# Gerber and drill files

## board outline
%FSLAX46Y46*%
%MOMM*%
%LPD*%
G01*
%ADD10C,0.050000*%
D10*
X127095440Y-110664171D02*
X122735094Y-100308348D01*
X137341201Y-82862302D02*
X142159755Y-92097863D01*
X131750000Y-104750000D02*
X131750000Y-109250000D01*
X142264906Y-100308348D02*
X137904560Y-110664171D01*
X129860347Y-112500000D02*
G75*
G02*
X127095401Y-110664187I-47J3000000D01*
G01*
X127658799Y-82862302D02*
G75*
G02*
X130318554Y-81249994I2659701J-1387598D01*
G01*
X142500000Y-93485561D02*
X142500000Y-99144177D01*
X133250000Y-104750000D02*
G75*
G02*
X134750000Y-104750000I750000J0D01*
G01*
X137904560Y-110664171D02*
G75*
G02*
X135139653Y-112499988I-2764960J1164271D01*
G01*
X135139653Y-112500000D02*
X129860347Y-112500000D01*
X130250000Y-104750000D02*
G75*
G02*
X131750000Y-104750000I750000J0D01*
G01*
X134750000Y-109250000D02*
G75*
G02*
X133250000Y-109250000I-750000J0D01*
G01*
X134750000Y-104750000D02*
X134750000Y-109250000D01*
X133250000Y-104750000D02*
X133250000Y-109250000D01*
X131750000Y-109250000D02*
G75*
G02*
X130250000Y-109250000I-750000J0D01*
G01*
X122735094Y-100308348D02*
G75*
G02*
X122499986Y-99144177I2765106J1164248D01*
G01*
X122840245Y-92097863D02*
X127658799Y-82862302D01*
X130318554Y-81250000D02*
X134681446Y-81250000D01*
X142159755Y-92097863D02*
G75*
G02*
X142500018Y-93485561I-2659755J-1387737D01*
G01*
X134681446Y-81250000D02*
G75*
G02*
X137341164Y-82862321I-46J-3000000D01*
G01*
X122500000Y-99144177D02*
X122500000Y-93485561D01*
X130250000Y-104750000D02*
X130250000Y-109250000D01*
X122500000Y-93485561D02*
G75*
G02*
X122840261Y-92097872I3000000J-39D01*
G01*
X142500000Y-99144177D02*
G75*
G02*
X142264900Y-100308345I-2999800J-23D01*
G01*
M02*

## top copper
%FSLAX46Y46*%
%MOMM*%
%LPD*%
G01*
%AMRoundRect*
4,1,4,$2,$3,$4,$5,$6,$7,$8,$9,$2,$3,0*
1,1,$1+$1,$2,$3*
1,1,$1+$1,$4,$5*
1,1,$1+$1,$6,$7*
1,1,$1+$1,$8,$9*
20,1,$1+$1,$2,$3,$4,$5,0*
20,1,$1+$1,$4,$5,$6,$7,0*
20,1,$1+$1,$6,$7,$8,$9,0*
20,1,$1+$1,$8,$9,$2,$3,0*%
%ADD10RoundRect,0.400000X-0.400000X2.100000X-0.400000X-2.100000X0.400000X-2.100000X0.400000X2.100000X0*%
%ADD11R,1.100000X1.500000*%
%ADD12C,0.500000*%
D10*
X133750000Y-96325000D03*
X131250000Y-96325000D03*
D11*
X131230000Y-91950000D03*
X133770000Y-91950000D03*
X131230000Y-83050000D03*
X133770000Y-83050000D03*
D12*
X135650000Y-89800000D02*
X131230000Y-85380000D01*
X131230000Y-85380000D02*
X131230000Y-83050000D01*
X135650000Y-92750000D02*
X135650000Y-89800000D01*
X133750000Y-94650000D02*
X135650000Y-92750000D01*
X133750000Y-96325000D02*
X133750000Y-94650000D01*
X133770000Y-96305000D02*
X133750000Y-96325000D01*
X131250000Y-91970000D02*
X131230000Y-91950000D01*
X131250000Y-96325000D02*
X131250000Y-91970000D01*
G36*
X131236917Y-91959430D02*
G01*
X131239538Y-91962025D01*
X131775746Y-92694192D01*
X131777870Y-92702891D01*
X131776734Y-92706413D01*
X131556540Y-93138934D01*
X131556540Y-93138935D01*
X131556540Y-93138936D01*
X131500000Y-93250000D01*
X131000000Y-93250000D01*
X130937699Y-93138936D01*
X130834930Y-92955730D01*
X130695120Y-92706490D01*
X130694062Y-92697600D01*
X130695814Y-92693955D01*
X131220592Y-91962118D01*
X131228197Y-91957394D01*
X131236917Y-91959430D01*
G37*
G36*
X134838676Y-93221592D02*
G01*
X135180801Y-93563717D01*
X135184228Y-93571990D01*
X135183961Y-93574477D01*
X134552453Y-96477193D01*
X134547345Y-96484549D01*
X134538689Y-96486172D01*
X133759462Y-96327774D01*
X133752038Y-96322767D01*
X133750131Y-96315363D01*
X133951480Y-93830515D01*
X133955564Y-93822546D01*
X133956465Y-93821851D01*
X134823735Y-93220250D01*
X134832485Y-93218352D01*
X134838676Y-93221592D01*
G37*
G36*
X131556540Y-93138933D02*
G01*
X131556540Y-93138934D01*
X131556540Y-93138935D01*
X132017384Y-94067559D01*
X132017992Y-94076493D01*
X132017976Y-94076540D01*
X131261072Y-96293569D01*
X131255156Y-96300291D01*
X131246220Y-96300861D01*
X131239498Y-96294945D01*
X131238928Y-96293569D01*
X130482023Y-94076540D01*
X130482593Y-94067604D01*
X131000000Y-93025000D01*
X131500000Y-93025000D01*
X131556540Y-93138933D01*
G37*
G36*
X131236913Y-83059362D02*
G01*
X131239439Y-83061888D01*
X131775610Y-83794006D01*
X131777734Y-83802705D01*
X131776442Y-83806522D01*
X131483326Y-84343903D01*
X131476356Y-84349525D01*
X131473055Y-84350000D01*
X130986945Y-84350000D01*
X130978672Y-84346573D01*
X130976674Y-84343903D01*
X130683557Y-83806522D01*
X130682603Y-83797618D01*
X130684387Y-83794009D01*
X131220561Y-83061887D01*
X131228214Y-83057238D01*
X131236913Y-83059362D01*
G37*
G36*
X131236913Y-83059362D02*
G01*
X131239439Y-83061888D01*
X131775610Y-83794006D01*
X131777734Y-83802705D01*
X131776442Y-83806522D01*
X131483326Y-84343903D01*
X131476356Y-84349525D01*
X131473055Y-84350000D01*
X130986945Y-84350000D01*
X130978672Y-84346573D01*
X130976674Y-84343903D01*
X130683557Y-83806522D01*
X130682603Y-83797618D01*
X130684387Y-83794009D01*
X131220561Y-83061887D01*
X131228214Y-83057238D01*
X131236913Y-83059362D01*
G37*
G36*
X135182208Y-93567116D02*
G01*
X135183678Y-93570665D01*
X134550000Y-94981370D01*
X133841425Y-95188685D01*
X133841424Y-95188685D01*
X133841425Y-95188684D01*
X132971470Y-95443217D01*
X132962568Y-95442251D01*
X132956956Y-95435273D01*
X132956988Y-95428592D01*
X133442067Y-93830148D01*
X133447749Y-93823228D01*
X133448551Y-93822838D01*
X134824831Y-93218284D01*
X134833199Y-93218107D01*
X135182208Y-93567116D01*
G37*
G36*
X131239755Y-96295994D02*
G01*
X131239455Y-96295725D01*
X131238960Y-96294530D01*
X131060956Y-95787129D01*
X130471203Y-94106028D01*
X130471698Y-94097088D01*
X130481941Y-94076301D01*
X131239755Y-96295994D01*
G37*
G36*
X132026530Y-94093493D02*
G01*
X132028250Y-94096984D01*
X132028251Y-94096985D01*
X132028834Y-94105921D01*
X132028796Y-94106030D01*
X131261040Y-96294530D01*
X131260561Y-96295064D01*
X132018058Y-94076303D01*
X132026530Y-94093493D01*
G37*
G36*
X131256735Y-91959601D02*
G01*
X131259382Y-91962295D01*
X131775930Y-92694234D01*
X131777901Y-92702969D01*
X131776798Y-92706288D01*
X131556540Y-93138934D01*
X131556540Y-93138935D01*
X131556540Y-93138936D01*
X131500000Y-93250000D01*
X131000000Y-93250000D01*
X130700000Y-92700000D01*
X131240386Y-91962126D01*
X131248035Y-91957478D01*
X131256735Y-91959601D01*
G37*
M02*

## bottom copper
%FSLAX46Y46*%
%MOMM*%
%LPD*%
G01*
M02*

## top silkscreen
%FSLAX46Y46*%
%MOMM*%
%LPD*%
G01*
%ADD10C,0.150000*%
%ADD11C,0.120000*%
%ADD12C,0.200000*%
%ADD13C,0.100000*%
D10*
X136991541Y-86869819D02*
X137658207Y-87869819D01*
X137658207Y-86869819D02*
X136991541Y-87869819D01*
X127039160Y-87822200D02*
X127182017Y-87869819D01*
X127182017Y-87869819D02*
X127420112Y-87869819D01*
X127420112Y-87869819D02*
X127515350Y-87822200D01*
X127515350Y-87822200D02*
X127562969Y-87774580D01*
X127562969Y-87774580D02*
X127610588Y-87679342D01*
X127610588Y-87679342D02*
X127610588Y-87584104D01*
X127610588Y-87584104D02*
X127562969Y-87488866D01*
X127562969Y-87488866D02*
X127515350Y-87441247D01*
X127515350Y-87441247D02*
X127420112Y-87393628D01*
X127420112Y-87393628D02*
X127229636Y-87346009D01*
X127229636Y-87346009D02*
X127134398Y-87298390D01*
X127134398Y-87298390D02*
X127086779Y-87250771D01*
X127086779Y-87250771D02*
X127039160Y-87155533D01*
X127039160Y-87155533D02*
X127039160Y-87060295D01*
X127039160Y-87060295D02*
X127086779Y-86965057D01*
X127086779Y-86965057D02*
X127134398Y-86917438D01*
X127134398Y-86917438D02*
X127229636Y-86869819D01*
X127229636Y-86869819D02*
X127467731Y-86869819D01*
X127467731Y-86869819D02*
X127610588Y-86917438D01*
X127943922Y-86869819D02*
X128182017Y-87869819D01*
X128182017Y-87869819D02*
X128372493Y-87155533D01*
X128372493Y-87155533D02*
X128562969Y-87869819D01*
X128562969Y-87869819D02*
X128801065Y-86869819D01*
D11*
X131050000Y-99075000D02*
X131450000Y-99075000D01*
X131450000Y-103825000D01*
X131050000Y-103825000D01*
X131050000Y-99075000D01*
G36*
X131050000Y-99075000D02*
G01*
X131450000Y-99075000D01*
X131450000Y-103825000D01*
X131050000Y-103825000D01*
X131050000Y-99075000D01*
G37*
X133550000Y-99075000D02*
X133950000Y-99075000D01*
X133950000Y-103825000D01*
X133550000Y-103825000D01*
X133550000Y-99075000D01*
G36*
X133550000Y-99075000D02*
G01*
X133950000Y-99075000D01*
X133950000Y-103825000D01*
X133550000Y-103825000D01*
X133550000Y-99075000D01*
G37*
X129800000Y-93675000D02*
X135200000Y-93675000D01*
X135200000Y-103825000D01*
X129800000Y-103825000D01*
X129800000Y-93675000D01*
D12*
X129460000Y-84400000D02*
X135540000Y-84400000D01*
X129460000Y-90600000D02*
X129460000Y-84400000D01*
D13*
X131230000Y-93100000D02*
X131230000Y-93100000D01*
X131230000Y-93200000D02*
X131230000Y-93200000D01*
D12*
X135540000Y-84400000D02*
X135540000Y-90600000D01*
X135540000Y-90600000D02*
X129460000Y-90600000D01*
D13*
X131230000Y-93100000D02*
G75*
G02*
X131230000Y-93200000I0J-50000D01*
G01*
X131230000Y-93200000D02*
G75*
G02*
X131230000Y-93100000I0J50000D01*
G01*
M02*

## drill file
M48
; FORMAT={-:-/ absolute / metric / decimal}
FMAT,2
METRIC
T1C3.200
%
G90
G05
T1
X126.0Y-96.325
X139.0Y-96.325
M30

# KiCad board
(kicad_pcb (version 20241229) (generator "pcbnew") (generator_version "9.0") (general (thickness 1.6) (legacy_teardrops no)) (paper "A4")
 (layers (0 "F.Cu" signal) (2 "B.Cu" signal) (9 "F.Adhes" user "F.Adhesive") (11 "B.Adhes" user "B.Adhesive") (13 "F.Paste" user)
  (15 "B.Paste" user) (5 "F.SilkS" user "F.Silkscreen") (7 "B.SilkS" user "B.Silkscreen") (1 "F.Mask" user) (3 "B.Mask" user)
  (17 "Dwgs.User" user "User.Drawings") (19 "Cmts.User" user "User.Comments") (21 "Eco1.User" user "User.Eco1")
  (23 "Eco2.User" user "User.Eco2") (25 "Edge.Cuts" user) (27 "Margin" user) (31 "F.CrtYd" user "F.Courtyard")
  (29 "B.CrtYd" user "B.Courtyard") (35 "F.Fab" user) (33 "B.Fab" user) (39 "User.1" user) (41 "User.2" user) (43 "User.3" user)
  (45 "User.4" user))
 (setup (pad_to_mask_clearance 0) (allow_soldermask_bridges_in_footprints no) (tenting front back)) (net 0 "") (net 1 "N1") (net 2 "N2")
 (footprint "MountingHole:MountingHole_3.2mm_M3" (layer "F.Cu") (at 139 96.325)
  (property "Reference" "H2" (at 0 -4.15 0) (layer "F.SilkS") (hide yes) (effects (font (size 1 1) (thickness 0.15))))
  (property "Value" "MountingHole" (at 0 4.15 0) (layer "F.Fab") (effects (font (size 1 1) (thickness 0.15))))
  (pad "" np_thru_hole circle (at 0 0) (size 3.2 3.2) (drill 3.2) (layers "*.Cu" "*.Mask")))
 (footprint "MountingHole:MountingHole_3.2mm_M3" (layer "F.Cu") (at 126 96.325)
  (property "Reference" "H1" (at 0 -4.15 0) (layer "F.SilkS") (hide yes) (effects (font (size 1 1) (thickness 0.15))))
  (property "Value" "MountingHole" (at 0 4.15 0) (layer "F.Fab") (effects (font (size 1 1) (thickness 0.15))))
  (pad "" np_thru_hole circle (at 0 0) (size 3.2 3.2) (drill 3.2) (layers "*.Cu" "*.Mask")))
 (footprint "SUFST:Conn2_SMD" (layer "F.Cu") (at 132.5 96.325 180)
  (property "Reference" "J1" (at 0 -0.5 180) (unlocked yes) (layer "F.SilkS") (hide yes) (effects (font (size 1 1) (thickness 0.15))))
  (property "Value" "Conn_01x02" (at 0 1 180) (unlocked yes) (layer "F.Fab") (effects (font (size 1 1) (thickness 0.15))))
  (fp_rect (start 1.05 -7.5) (end 1.45 -2.75) (stroke (width 0.12) (type solid)) (fill yes) (layer "F.SilkS"))
  (fp_rect (start -1.45 -7.5) (end -1.05 -2.75) (stroke (width 0.12) (type solid)) (fill yes) (layer "F.SilkS"))
  (fp_rect (start -2.7 -7.5) (end 2.7 2.65) (stroke (width 0.12) (type default)) (fill no) (layer "F.SilkS"))
  (pad "1" smd roundrect (at -1.25 0 270) (size 5 1.6) (layers "F.Cu" "F.Mask" "F.Paste") (roundrect_rratio 0.25) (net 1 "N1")
   (thermal_bridge_angle 45)
   (teardrops (best_length_ratio 0.5) (max_length 1) (best_width_ratio 1) (max_width 2) (curved_edges no) (filter_ratio 0.9) (enabled yes)
    (allow_two_segments yes) (prefer_zone_connections yes)))
  (pad "2" smd roundrect (at 1.25 0 270) (size 5 1.6) (layers "F.Cu" "F.Mask" "F.Paste") (roundrect_rratio 0.25) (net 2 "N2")
   (thermal_bridge_angle 45)
   (teardrops (best_length_ratio 0.5) (max_length 1) (best_width_ratio 1) (max_width 2) (curved_edges no) (filter_ratio 0.9) (enabled yes)
    (allow_two_segments yes) (prefer_zone_connections yes))))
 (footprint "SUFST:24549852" (layer "F.Cu") (at 132.5 87.5)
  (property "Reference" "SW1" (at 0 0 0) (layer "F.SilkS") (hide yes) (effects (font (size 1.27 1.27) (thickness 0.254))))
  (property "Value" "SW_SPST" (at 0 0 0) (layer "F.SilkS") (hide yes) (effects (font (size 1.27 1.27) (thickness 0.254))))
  (fp_line (start -3.04 -3.1) (end 3.04 -3.1) (stroke (width 0.2) (type solid)) (layer "F.SilkS"))
  (fp_line (start -3.04 3.1) (end -3.04 -3.1) (stroke (width 0.2) (type solid)) (layer "F.SilkS"))
  (fp_line (start -1.27 5.6) (end -1.27 5.6) (stroke (width 0.1) (type solid)) (layer "F.SilkS"))
  (fp_line (start -1.27 5.7) (end -1.27 5.7) (stroke (width 0.1) (type solid)) (layer "F.SilkS"))
  (fp_line (start 3.04 -3.1) (end 3.04 3.1) (stroke (width 0.2) (type solid)) (layer "F.SilkS"))
  (fp_line (start 3.04 3.1) (end -3.04 3.1) (stroke (width 0.2) (type solid)) (layer "F.SilkS"))
  (fp_arc (start -1.27 5.6) (mid -1.22 5.65) (end -1.27 5.7) (stroke (width 0.1) (type solid)) (layer "F.SilkS"))
  (fp_arc (start -1.27 5.7) (mid -1.32 5.65) (end -1.27 5.6) (stroke (width 0.1) (type solid)) (layer "F.SilkS"))
  (pad "A1" smd rect (at -1.27 4.45) (size 1.1 1.5) (layers "F.Cu" "F.Mask" "F.Paste") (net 2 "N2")
   (teardrops (best_length_ratio 0.5) (max_length 1) (best_width_ratio 1) (max_width 2) (curved_edges no) (filter_ratio 0.9) (enabled yes)
    (allow_two_segments yes) (prefer_zone_connections yes)))
  (pad "A2" smd rect (at 1.27 4.45) (size 1.1 1.5) (layers "F.Cu" "F.Mask" "F.Paste")
   (teardrops (best_length_ratio 0.5) (max_length 1) (best_width_ratio 1) (max_width 2) (curved_edges no) (filter_ratio 0.9) (enabled yes)
    (allow_two_segments yes) (prefer_zone_connections yes)))
  (pad "B1" smd rect (at -1.27 -4.45) (size 1.1 1.5) (layers "F.Cu" "F.Mask" "F.Paste") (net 1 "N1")
   (teardrops (best_length_ratio 0.5) (max_length 1) (best_width_ratio 1) (max_width 2) (curved_edges no) (filter_ratio 0.9) (enabled yes)
    (allow_two_segments yes) (prefer_zone_connections yes)))
  (pad "B2" smd rect (at 1.27 -4.45) (size 1.1 1.5) (layers "F.Cu" "F.Mask" "F.Paste")
   (teardrops (best_length_ratio 0.5) (max_length 1) (best_width_ratio 1) (max_width 2) (curved_edges no) (filter_ratio 0.9) (enabled yes)
    (allow_two_segments yes) (prefer_zone_connections yes))))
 (gr_line (start 127.09544 110.664171) (end 122.735094 100.308348) (stroke (width 0.05) (type default)) (layer "Edge.Cuts"))
 (gr_line (start 137.341201 82.862302) (end 142.159755 92.097863) (stroke (width 0.05) (type default)) (layer "Edge.Cuts"))
 (gr_line (start 131.75 104.75) (end 131.75 109.25) (stroke (width 0.05) (type default)) (layer "Edge.Cuts"))
 (gr_line (start 142.264906 100.308348) (end 137.90456 110.664171) (stroke (width 0.05) (type default)) (layer "Edge.Cuts"))
 (gr_arc (start 129.860347 112.5) (mid 128.200906 111.999251) (end 127.09544 110.664171) (stroke (width 0.05) (type default))
  (layer "Edge.Cuts"))
 (gr_arc (start 127.658799 82.862302) (mid 128.763412 81.68453) (end 130.318554 81.25) (stroke (width 0.05) (type default))
  (layer "Edge.Cuts"))
 (gr_line (start 142.5 93.485561) (end 142.5 99.144177) (stroke (width 0.05) (type default)) (layer "Edge.Cuts"))
 (gr_arc (start 133.25 104.75) (mid 134 104) (end 134.75 104.75) (stroke (width 0.05) (type default)) (layer "Edge.Cuts"))
 (gr_arc (start 137.90456 110.664171) (mid 136.79909 111.999234) (end 135.139653 112.5) (stroke (width 0.05) (type default))
  (layer "Edge.Cuts"))
 (gr_line (start 135.139653 112.5) (end 129.860347 112.5) (stroke (width 0.05) (type default)) (layer "Edge.Cuts"))
 (gr_arc (start 130.25 104.75) (mid 131 104) (end 131.75 104.75) (stroke (width 0.05) (type default)) (layer "Edge.Cuts"))
 (gr_arc (start 134.75 109.25) (mid 134 110) (end 133.25 109.25) (stroke (width 0.05) (type default)) (layer "Edge.Cuts"))
 (gr_line (start 134.75 104.75) (end 134.75 109.25) (stroke (width 0.05) (type default)) (layer "Edge.Cuts"))
 (gr_line (start 133.25 104.75) (end 133.25 109.25) (stroke (width 0.05) (type default)) (layer "Edge.Cuts"))
 (gr_arc (start 131.75 109.25) (mid 131 110) (end 130.25 109.25) (stroke (width 0.05) (type default)) (layer "Edge.Cuts"))
 (gr_arc (start 122.735094 100.308348) (mid 122.559365 99.738012) (end 122.5 99.144177) (stroke (width 0.05) (type default))
  (layer "Edge.Cuts"))
 (gr_line (start 122.840245 92.097863) (end 127.658799 82.862302) (stroke (width 0.05) (type default)) (layer "Edge.Cuts"))
 (gr_line (start 130.318554 81.25) (end 134.681446 81.25) (stroke (width 0.05) (type default)) (layer "Edge.Cuts"))
 (gr_arc (start 142.159755 92.097863) (mid 142.413698 92.77116) (end 142.5 93.485561) (stroke (width 0.05) (type default))
  (layer "Edge.Cuts"))
 (gr_arc (start 134.681446 81.25) (mid 136.236584 81.684547) (end 137.341201 82.862302) (stroke (width 0.05) (type default))
  (layer "Edge.Cuts"))
 (gr_line (start 122.5 99.144177) (end 122.5 93.485561) (stroke (width 0.05) (type default)) (layer "Edge.Cuts"))
 (gr_line (start 130.25 104.75) (end 130.25 109.25) (stroke (width 0.05) (type default)) (layer "Edge.Cuts"))
 (gr_arc (start 122.5 93.485561) (mid 122.586303 92.771161) (end 122.840245 92.097863) (stroke (width 0.05) (type default))
  (layer "Edge.Cuts"))
 (gr_arc (start 142.5 99.144177) (mid 142.440644 99.738014) (end 142.264906 100.308348) (stroke (width 0.05) (type default))
  (layer "Edge.Cuts"))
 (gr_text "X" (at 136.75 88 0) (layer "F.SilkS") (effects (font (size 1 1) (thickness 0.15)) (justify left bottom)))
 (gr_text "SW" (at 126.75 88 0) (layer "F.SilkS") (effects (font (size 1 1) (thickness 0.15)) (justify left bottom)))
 (segment (start 135.65 89.8) (end 131.23 85.38) (width 0.5) (layer "F.Cu") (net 1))
 (segment (start 131.23 85.38) (end 131.23 83.05) (width 0.5) (layer "F.Cu") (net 1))
 (segment (start 135.65 92.75) (end 135.65 89.8) (width 0.5) (layer "F.Cu") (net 1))
 (segment (start 133.75 94.65) (end 135.65 92.75) (width 0.5) (layer "F.Cu") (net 1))
 (segment (start 133.75 96.325) (end 133.75 94.65) (width 0.5) (layer "F.Cu") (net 1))
 (segment (start 133.77 96.305) (end 133.75 96.325) (width 0.5) (layer "F.Cu") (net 1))
 (segment (start 131.25 91.97) (end 131.23 91.95) (width 0.5) (layer "F.Cu") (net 2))
 (segment (start 131.25 96.325) (end 131.25 91.97) (width 0.5) (layer "F.Cu") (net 2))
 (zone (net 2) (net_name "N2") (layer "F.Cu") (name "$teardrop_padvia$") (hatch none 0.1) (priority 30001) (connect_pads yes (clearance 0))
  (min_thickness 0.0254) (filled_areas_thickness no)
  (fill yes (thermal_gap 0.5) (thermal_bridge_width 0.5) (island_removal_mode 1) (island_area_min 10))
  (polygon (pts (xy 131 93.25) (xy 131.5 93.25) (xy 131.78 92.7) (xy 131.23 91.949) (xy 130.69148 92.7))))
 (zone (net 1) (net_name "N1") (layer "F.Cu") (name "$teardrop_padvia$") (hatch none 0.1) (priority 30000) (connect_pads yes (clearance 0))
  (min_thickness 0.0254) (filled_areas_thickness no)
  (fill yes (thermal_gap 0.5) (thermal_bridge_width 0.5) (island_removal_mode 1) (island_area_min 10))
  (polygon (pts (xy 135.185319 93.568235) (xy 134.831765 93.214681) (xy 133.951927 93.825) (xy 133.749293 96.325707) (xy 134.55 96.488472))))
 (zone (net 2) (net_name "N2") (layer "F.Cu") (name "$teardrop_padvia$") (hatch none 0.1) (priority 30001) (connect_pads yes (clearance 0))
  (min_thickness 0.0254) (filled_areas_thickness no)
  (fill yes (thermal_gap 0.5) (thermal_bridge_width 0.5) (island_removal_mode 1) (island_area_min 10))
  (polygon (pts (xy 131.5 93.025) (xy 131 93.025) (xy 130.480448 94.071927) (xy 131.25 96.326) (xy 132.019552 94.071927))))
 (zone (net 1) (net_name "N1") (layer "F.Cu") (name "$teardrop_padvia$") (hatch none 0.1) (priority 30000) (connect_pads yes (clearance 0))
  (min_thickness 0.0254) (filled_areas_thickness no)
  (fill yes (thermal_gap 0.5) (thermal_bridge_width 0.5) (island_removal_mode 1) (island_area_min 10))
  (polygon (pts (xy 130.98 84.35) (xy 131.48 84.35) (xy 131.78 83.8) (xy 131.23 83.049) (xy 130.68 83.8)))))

